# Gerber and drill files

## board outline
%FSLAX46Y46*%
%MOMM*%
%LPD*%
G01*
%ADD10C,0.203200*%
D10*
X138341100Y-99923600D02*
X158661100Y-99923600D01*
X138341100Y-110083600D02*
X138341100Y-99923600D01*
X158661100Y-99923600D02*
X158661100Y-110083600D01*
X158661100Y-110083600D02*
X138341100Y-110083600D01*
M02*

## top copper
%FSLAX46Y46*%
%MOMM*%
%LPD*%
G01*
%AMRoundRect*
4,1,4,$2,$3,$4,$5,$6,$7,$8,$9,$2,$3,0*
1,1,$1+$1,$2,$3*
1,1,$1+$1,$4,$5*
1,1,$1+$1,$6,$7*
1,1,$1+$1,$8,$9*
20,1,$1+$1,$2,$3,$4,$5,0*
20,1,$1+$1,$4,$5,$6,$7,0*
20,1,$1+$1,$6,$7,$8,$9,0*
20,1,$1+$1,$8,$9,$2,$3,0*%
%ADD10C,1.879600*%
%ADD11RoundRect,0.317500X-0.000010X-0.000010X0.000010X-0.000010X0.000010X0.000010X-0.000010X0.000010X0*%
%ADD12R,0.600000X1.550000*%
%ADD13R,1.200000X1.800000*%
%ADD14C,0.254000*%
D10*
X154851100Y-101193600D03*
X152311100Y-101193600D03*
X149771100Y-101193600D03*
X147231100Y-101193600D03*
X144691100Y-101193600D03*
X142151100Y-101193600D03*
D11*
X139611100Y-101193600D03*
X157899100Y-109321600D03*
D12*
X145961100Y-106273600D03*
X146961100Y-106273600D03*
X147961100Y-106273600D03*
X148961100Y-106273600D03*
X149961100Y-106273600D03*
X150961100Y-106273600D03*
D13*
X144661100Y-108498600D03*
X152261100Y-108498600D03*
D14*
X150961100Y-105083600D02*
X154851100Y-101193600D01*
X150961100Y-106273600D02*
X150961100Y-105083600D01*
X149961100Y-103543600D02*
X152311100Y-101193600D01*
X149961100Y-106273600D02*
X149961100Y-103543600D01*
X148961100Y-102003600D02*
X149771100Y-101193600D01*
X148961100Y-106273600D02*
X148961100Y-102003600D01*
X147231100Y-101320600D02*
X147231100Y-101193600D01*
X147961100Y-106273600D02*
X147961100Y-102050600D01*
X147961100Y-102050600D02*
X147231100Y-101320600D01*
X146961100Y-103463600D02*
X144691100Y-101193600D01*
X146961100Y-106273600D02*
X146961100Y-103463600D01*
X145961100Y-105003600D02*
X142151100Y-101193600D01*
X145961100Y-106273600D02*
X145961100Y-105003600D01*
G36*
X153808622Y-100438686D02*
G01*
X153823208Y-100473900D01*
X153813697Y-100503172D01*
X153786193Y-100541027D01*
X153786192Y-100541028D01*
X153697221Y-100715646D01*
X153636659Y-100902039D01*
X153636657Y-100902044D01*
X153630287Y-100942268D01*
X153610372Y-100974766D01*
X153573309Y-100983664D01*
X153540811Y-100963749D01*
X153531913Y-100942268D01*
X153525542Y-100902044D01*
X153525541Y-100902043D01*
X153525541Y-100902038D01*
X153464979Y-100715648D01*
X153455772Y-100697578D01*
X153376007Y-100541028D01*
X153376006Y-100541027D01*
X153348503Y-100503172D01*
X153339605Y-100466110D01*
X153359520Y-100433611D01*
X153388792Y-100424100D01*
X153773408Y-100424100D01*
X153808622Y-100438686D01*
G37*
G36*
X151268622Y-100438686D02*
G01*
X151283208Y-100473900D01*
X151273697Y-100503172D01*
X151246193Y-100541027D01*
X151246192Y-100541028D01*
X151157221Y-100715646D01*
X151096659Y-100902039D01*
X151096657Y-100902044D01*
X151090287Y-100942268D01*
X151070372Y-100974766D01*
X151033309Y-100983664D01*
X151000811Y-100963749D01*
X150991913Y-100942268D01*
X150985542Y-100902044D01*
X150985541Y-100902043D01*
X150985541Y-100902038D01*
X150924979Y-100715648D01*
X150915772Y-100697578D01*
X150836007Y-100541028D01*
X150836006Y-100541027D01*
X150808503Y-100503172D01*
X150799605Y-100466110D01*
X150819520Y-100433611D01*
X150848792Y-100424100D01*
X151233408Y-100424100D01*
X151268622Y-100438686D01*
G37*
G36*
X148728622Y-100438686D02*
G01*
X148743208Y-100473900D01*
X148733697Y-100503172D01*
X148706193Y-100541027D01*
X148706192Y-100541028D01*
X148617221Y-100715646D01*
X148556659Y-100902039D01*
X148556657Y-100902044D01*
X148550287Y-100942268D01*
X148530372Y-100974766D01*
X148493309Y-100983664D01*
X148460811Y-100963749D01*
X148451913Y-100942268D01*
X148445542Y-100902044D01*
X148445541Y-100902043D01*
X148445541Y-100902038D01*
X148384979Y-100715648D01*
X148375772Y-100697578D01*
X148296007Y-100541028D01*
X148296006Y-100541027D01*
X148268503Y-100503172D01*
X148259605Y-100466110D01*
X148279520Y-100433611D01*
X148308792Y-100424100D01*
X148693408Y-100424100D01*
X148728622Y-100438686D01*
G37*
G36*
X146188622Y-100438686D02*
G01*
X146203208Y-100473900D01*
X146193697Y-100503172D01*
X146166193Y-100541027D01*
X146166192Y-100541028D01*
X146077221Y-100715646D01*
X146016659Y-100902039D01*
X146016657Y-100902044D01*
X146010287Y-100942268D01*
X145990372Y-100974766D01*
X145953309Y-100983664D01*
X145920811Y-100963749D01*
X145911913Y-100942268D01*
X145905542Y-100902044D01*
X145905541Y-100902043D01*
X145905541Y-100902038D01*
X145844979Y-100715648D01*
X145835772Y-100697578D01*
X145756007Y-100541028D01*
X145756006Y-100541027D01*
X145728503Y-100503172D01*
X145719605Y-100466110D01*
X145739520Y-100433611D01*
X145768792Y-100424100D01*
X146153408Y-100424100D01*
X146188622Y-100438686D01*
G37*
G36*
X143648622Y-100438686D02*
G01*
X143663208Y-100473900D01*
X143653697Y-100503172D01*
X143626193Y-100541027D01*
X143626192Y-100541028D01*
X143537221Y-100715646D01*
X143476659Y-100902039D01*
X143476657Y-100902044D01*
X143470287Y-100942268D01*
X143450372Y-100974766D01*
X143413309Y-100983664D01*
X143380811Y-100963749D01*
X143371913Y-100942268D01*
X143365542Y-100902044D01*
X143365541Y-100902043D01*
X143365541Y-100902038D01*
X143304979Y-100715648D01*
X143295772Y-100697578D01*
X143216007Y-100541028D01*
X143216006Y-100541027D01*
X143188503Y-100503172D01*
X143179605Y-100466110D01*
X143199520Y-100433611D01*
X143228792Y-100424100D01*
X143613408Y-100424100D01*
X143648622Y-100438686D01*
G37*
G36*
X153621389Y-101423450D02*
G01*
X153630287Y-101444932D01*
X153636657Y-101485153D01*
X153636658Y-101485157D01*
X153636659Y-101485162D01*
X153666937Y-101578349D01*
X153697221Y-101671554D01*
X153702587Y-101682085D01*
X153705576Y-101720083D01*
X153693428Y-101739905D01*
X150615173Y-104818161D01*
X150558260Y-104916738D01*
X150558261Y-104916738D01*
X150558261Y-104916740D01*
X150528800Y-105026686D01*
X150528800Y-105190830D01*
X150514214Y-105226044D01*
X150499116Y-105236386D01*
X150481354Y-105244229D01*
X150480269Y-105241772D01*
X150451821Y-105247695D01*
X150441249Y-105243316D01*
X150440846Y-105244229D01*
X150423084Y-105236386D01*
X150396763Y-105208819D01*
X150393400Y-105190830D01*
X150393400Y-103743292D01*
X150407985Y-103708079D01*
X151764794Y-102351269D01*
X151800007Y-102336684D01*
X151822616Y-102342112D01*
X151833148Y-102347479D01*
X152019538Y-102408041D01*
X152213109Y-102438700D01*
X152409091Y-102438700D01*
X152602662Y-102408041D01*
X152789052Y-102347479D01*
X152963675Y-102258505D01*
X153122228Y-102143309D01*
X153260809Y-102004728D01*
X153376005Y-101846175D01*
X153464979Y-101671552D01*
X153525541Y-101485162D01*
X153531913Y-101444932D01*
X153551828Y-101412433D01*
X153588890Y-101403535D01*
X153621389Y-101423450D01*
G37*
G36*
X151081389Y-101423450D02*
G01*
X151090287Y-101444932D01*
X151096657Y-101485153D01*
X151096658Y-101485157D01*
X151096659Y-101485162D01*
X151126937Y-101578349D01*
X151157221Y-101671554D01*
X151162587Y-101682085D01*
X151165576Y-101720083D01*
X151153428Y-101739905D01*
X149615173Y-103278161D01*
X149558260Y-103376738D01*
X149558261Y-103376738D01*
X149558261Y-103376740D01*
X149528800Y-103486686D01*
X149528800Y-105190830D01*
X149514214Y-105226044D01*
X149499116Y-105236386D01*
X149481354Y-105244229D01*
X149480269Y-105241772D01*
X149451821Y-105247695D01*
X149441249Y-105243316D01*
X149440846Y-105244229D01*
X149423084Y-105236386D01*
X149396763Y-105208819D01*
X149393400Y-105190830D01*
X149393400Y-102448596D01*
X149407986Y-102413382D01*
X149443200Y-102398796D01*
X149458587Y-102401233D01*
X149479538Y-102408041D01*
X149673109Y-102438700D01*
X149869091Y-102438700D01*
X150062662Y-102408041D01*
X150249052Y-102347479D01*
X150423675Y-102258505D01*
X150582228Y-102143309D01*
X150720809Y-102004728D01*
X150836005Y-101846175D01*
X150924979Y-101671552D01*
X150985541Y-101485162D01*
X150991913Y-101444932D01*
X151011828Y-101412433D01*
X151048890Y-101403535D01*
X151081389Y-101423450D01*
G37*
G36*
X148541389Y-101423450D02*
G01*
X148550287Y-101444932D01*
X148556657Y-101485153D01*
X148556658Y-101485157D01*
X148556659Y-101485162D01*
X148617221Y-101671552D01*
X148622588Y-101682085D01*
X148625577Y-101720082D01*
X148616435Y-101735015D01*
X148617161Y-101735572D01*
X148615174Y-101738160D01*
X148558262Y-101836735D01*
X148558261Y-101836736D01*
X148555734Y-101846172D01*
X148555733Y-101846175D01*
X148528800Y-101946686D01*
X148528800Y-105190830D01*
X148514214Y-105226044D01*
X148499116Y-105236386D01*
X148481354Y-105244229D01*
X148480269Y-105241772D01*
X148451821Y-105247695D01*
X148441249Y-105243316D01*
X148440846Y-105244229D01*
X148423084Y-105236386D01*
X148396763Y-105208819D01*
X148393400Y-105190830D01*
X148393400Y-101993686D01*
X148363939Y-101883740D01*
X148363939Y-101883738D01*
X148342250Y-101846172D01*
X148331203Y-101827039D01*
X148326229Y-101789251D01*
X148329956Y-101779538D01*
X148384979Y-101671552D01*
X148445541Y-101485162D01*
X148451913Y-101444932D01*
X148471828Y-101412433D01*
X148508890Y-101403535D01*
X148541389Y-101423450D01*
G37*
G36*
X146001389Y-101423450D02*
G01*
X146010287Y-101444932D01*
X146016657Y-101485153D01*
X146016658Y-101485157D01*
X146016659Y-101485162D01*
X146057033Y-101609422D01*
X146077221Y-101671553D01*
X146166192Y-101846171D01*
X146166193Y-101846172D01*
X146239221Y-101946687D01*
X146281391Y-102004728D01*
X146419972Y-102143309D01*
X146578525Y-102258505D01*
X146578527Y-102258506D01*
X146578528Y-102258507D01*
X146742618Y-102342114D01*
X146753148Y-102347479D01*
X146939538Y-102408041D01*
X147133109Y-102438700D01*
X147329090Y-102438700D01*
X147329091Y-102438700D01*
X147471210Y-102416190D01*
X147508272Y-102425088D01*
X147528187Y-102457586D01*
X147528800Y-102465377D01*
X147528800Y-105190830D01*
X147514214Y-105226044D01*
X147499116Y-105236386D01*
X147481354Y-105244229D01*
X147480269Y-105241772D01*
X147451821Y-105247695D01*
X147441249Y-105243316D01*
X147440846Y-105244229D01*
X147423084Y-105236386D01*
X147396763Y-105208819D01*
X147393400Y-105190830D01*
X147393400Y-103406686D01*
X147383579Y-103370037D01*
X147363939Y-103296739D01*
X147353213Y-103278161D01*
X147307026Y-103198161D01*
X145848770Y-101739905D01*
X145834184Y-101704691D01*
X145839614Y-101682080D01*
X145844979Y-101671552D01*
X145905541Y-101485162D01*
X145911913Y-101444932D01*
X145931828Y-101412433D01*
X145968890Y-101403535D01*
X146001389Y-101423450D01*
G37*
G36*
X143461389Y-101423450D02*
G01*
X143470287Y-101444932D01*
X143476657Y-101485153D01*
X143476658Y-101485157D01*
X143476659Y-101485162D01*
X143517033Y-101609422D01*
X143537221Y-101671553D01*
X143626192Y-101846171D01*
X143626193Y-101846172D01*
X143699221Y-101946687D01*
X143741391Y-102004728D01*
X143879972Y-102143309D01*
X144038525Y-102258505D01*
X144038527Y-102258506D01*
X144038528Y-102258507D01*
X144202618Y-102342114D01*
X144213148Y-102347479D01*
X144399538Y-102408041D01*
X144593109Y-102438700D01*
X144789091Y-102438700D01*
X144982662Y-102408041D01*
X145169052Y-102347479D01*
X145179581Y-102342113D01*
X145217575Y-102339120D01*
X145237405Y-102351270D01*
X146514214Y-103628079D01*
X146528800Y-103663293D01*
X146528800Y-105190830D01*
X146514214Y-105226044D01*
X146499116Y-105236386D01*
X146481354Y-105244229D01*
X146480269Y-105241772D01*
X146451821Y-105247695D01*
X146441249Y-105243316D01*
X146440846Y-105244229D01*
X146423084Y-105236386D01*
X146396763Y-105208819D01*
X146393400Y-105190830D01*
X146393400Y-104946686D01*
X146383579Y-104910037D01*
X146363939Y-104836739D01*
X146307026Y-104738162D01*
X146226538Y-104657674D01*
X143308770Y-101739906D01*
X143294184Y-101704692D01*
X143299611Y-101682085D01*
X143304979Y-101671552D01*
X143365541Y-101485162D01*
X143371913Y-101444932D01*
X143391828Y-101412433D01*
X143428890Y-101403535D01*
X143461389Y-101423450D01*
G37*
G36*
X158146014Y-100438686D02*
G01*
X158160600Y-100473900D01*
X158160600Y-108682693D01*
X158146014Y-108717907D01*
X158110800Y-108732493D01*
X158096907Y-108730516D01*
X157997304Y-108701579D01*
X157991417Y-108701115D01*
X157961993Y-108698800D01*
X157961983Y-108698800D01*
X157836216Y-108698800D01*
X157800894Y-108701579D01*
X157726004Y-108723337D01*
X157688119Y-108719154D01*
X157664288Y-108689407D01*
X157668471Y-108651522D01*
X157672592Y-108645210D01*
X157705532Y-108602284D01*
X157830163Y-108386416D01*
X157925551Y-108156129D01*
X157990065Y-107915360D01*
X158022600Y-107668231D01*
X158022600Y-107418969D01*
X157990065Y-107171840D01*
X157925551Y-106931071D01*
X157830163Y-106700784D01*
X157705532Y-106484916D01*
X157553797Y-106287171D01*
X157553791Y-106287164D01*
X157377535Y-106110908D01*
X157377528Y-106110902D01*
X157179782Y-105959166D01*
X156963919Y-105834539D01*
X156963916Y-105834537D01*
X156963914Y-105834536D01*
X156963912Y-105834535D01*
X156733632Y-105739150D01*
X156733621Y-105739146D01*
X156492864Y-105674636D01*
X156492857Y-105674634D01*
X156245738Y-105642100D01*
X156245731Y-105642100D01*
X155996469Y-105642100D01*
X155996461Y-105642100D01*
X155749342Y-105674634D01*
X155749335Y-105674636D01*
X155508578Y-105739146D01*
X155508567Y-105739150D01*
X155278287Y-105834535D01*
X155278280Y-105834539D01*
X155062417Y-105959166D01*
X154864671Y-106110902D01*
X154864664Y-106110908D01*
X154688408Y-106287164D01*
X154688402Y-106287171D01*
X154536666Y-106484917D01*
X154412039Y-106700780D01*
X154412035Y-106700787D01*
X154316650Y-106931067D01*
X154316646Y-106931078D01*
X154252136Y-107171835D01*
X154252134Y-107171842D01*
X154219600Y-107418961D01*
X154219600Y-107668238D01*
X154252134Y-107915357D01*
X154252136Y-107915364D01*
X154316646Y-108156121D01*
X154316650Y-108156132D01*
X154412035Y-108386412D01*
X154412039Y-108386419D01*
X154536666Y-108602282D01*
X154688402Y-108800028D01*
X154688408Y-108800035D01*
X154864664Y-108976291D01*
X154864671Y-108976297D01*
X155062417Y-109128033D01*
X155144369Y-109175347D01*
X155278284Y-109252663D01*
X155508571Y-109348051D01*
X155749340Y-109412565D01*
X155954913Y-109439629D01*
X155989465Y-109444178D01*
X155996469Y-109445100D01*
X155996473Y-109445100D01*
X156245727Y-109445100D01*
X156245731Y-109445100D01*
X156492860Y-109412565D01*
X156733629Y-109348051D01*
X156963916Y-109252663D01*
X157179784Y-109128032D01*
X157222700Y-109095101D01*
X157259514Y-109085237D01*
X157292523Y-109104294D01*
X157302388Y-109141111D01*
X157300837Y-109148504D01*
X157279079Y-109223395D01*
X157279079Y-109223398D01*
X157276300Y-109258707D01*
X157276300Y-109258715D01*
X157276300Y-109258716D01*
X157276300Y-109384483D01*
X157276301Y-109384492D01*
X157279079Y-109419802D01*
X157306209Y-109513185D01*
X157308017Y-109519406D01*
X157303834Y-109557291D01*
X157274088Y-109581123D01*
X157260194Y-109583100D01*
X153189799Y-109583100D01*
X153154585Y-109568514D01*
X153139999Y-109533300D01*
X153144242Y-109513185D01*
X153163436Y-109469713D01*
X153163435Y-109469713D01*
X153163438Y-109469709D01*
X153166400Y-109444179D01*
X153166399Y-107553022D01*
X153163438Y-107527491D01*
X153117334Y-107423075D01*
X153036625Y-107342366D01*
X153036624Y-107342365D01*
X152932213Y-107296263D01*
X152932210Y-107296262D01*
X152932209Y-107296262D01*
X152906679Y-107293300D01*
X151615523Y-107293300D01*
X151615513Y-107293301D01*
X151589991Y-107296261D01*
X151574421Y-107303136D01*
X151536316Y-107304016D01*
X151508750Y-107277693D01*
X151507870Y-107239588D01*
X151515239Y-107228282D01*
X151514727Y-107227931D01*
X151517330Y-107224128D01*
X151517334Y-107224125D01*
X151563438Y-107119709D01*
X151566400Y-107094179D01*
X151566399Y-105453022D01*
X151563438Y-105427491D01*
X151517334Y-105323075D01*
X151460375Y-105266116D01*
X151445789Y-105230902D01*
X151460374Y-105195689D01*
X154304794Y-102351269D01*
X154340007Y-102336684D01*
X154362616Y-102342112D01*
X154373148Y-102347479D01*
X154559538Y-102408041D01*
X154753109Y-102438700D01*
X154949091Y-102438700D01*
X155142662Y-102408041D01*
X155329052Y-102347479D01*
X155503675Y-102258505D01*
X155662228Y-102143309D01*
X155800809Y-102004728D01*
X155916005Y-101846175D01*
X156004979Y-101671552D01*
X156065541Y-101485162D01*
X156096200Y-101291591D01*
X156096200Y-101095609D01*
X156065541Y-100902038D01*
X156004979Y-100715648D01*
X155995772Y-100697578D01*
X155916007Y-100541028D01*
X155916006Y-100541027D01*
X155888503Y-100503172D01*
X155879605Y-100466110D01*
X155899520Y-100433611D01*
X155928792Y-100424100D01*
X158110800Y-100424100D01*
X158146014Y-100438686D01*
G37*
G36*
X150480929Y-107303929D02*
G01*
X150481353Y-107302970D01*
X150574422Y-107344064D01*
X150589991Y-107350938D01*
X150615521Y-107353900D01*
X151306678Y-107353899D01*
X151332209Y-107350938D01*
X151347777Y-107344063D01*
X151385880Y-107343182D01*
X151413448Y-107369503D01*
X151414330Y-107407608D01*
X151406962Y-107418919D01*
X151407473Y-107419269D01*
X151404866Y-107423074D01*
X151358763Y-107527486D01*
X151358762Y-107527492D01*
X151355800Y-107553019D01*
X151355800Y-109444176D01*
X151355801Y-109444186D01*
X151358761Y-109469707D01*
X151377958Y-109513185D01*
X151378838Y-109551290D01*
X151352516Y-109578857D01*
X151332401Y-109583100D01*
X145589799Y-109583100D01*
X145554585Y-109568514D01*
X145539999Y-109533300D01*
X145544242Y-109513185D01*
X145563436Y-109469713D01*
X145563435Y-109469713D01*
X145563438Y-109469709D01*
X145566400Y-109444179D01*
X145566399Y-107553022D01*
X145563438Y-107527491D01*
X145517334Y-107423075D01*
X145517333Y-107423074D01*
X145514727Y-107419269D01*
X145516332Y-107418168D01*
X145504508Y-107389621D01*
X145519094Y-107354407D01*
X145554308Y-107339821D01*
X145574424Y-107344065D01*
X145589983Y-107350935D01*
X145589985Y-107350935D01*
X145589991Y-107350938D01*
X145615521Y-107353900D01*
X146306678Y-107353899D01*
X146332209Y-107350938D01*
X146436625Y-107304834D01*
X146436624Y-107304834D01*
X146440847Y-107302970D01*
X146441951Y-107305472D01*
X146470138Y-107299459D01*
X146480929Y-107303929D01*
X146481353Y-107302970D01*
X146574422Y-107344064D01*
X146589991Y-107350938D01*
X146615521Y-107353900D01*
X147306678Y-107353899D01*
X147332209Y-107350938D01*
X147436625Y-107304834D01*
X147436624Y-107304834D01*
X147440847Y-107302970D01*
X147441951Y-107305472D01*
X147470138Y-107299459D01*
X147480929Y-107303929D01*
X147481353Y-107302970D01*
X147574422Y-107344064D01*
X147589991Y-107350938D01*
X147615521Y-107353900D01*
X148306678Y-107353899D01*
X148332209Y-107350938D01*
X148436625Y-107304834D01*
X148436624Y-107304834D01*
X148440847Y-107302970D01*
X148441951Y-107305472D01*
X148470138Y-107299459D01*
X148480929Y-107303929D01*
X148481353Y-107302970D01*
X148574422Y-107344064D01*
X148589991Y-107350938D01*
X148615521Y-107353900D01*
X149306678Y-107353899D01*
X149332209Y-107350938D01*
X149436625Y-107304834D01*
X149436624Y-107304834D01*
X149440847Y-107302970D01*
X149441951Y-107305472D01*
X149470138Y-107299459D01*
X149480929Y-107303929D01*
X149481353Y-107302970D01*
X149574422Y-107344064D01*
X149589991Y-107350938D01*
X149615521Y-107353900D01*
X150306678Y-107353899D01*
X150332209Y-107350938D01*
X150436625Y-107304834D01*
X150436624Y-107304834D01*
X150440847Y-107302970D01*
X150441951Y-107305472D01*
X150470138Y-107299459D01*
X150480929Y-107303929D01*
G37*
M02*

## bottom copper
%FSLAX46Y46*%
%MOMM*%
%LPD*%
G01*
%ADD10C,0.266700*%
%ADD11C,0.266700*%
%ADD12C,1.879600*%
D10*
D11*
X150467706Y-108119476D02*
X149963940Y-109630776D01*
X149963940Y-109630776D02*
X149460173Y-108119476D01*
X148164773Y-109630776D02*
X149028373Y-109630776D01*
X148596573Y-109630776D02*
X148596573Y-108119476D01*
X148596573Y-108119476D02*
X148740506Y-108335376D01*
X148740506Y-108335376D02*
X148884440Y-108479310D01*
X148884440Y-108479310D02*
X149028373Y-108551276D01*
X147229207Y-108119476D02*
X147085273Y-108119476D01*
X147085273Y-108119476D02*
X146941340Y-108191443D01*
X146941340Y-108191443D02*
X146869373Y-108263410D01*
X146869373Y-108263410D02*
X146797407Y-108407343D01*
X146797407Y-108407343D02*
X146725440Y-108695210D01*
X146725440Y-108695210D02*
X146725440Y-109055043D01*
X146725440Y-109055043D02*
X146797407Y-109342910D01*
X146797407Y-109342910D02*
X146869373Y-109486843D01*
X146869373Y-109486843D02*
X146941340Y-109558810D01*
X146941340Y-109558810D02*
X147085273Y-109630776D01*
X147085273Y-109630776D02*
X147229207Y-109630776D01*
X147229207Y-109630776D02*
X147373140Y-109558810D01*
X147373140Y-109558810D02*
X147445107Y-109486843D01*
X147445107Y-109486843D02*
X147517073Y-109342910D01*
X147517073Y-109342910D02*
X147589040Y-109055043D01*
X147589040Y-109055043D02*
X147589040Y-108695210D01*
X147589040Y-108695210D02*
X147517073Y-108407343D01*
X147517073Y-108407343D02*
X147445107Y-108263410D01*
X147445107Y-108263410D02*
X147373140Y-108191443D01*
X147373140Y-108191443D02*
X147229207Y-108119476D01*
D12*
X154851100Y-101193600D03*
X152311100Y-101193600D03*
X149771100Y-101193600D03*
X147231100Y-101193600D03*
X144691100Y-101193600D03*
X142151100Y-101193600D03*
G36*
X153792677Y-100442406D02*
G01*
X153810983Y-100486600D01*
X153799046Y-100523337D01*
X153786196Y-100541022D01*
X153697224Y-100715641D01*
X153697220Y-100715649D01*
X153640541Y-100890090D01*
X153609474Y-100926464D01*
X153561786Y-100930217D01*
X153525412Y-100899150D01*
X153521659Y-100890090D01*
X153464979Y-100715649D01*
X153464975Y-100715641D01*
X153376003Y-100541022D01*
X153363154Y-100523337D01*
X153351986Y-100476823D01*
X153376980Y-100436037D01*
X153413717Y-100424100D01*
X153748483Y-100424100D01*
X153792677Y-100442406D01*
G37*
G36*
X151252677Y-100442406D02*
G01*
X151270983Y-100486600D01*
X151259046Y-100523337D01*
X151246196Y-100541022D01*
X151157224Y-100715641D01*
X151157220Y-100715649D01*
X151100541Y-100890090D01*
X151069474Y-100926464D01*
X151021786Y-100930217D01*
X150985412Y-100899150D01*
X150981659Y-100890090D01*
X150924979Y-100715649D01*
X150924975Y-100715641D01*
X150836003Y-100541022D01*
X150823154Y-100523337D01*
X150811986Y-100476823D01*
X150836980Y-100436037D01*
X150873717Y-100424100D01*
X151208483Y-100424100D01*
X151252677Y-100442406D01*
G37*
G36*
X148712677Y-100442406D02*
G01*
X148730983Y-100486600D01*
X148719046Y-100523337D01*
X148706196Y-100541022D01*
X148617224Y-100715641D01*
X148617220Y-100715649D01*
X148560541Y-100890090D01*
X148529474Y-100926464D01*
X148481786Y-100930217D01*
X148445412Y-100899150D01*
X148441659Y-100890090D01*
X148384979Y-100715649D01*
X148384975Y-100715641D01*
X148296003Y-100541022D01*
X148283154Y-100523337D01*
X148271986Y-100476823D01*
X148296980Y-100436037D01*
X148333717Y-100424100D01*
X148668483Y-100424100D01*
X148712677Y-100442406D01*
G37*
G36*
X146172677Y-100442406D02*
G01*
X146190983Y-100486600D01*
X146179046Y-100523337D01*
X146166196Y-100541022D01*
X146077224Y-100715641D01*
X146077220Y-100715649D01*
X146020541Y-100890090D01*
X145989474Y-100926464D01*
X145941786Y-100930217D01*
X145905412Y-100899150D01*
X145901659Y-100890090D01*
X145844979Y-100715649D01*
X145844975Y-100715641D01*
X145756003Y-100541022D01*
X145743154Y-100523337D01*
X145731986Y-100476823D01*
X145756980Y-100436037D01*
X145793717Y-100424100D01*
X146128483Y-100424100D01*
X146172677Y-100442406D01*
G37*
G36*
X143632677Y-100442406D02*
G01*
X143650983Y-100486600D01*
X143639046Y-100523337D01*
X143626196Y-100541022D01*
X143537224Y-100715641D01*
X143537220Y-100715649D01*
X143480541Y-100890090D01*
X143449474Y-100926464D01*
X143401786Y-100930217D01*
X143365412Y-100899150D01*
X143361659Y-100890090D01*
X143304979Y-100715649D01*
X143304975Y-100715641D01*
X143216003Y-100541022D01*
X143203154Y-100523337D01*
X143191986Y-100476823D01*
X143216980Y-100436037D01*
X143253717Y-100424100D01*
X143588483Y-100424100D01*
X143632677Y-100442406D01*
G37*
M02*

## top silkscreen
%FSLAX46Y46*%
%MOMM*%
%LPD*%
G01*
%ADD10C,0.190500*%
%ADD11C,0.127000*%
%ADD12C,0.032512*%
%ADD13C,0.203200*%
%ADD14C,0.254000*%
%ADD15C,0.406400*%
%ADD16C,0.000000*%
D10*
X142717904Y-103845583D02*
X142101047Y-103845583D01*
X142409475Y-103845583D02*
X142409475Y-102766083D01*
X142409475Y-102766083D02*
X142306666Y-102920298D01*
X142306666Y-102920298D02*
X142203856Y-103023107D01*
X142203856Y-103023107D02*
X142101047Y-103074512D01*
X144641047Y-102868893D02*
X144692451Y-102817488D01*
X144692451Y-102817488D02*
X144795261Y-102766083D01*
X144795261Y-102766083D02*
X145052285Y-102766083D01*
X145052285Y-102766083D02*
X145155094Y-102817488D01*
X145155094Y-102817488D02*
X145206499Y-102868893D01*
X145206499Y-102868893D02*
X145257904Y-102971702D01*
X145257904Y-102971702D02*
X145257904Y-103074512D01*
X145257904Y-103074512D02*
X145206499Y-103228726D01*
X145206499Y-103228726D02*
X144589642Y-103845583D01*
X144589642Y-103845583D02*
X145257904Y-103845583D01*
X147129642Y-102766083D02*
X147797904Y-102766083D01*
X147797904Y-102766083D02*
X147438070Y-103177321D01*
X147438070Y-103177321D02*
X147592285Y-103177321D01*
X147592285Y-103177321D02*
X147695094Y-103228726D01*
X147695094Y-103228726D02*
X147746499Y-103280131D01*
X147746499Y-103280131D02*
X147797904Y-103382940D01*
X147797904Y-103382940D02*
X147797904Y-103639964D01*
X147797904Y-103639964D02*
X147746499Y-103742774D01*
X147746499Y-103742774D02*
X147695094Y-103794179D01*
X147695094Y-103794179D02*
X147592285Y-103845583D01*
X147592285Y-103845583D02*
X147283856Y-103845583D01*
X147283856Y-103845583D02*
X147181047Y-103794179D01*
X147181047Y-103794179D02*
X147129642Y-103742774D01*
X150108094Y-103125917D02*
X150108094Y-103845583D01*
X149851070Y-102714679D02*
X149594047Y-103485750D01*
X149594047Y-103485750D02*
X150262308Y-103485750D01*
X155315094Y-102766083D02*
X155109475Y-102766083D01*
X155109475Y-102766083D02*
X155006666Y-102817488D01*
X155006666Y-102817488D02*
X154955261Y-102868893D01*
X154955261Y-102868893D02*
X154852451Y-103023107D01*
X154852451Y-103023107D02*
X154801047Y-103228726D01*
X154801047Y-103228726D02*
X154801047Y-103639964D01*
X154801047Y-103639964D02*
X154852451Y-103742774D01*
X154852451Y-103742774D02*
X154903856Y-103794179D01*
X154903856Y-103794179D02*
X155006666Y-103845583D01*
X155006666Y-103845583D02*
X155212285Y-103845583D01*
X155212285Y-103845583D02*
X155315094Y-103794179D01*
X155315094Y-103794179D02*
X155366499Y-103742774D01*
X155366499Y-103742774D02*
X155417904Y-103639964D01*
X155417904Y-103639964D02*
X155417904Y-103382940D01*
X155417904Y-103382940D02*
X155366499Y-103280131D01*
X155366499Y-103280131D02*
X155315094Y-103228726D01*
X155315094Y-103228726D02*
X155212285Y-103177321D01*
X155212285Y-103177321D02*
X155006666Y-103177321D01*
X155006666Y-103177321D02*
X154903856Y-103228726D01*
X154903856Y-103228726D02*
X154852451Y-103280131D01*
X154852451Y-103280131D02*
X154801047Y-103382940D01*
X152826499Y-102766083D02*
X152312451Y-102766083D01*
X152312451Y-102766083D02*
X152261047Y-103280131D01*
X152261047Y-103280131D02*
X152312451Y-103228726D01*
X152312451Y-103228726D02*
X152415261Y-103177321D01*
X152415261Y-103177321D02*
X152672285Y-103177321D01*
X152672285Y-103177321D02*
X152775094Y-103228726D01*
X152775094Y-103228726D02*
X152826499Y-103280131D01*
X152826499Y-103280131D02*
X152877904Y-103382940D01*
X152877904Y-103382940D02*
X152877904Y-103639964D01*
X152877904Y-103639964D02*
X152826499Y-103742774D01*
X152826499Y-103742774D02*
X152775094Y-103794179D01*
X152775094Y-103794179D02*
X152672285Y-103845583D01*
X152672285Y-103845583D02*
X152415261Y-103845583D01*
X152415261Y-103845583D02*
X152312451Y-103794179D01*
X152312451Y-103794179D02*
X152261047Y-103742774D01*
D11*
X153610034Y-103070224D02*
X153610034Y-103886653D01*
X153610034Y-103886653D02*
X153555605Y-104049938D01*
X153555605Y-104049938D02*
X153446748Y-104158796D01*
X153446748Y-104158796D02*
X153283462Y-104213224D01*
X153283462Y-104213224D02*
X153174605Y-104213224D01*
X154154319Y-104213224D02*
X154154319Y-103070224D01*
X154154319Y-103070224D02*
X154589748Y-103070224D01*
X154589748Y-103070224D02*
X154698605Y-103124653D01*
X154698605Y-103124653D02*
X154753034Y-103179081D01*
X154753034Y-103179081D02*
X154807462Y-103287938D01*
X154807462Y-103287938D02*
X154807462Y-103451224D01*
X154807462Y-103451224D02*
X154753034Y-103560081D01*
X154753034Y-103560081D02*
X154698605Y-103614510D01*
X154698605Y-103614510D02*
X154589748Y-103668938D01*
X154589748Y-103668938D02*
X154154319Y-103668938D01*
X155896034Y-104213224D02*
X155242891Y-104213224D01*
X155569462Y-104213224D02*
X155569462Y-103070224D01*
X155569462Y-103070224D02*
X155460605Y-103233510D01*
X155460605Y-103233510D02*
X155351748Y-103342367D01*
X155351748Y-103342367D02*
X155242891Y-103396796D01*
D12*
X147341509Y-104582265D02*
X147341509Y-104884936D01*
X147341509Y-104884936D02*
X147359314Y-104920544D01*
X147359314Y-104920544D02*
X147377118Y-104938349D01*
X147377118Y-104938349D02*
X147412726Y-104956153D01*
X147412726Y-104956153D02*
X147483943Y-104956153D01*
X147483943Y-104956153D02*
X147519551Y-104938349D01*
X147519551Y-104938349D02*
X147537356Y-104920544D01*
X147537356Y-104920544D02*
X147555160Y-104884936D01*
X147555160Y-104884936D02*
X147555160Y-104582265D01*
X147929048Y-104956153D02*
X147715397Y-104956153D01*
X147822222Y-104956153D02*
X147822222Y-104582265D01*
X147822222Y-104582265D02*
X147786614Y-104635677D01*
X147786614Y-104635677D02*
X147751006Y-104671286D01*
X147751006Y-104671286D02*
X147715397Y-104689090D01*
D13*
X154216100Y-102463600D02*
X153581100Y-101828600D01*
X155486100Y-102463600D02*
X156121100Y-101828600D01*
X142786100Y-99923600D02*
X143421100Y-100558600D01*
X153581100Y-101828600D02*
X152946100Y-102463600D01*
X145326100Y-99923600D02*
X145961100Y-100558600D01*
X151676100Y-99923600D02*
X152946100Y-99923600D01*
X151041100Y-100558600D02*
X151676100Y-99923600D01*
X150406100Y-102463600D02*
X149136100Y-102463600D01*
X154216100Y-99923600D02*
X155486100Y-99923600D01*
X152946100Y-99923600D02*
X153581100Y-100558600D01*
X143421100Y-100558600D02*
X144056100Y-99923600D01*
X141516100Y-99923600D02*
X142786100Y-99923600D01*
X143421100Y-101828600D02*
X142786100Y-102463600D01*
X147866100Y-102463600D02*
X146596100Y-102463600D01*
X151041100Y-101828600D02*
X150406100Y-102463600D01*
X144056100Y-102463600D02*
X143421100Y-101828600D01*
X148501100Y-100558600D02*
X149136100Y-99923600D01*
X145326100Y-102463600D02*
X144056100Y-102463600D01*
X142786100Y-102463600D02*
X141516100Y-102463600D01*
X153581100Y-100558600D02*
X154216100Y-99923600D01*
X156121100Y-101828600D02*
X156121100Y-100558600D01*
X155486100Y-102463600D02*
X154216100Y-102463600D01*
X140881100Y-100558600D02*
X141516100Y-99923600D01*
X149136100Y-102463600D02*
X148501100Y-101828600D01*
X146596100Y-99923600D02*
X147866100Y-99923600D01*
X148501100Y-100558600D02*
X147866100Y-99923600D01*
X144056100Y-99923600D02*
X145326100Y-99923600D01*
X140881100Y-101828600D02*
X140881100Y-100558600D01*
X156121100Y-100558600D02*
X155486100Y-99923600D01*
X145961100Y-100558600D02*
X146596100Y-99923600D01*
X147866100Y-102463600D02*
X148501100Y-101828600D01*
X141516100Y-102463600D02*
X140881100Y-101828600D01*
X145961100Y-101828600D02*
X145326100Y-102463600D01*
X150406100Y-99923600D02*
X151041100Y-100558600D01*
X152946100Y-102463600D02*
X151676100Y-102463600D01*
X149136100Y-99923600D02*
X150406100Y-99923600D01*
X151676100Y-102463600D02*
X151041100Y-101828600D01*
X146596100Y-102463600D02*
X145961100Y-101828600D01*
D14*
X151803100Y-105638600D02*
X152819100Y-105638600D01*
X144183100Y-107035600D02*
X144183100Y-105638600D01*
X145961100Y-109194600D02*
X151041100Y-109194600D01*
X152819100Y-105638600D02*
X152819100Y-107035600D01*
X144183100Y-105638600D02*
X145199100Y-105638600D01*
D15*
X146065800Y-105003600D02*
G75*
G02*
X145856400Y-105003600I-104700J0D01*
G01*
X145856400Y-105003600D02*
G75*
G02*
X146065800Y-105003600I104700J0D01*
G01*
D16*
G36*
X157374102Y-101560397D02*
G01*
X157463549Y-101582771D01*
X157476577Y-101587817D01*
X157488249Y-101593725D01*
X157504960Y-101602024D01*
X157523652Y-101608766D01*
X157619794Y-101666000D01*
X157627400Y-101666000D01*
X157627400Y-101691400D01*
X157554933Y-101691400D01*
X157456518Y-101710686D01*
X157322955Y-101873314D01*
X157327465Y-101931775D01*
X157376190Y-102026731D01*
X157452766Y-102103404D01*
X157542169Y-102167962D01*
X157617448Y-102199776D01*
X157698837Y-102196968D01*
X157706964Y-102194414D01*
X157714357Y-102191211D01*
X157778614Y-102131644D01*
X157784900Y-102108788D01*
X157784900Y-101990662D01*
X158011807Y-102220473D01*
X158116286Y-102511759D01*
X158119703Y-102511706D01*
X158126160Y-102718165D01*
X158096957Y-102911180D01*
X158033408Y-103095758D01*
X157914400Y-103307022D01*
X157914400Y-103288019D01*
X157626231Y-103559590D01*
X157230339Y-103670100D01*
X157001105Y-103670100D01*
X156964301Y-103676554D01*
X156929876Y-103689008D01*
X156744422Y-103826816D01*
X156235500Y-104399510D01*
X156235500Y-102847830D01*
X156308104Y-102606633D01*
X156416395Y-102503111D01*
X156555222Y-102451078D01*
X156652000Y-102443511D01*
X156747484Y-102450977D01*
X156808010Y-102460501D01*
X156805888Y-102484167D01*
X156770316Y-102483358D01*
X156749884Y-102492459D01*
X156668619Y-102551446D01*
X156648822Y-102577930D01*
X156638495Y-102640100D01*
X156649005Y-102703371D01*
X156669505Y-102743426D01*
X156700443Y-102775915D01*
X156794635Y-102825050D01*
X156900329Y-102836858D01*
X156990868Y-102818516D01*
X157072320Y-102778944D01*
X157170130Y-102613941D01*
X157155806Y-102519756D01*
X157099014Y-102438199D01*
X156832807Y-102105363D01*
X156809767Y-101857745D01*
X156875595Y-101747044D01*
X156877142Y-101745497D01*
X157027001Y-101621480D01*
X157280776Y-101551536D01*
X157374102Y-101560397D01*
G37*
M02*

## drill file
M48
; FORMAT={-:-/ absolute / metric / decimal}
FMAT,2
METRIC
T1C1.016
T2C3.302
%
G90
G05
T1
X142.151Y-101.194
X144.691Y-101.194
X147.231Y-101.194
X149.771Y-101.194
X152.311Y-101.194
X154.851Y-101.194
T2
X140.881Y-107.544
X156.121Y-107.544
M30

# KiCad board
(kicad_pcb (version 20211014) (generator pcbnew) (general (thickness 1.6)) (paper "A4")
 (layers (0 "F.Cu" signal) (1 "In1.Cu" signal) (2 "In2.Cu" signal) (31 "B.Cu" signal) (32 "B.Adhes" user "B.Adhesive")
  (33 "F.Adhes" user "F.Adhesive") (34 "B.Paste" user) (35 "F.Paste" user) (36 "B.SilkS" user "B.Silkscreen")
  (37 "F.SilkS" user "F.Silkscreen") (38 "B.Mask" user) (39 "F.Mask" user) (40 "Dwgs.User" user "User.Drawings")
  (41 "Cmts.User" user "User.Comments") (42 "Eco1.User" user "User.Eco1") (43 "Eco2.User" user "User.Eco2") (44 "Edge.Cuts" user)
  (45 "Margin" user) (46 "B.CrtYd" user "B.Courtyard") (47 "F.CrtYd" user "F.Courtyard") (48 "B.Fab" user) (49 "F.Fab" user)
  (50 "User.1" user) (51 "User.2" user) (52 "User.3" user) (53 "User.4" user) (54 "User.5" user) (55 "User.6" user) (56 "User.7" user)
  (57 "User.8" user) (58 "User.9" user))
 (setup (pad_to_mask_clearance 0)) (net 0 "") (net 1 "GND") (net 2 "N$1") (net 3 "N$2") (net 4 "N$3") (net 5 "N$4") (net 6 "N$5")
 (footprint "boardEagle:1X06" (layer "F.Cu") (at 154.8511 101.1936 180)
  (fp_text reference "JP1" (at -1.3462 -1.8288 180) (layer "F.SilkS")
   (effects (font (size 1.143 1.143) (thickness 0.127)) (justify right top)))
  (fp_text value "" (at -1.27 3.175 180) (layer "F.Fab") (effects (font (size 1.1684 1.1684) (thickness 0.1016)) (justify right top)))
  (fp_line (start 0.635 -1.27) (end 1.27 -0.635) (layer "F.SilkS") (width 0.2032))
  (fp_line (start -0.635 -1.27) (end -1.27 -0.635) (layer "F.SilkS") (width 0.2032))
  (fp_line (start 12.065 1.27) (end 11.43 0.635) (layer "F.SilkS") (width 0.2032))
  (fp_line (start 1.27 -0.635) (end 1.905 -1.27) (layer "F.SilkS") (width 0.2032))
  (fp_line (start 9.525 1.27) (end 8.89 0.635) (layer "F.SilkS") (width 0.2032))
  (fp_line (start 3.175 1.27) (end 1.905 1.27) (layer "F.SilkS") (width 0.2032))
  (fp_line (start 3.81 0.635) (end 3.175 1.27) (layer "F.SilkS") (width 0.2032))
  (fp_line (start 4.445 -1.27) (end 5.715 -1.27) (layer "F.SilkS") (width 0.2032))
  (fp_line (start 0.635 1.27) (end -0.635 1.27) (layer "F.SilkS") (width 0.2032))
  (fp_line (start 1.905 1.27) (end 1.27 0.635) (layer "F.SilkS") (width 0.2032))
  (fp_line (start 11.43 0.635) (end 10.795 1.27) (layer "F.SilkS") (width 0.2032))
  (fp_line (start 13.335 1.27) (end 12.065 1.27) (layer "F.SilkS") (width 0.2032))
  (fp_line (start 11.43 -0.635) (end 12.065 -1.27) (layer "F.SilkS") (width 0.2032))
  (fp_line (start 6.985 -1.27) (end 8.255 -1.27) (layer "F.SilkS") (width 0.2032))
  (fp_line (start 3.81 -0.635) (end 4.445 -1.27) (layer "F.SilkS") (width 0.2032))
  (fp_line (start 10.795 -1.27) (end 11.43 -0.635) (layer "F.SilkS") (width 0.2032))
  (fp_line (start 6.35 0.635) (end 5.715 1.27) (layer "F.SilkS") (width 0.2032))
  (fp_line (start 9.525 -1.27) (end 10.795 -1.27) (layer "F.SilkS") (width 0.2032))
  (fp_line (start 12.065 -1.27) (end 13.335 -1.27) (layer "F.SilkS") (width 0.2032))
  (fp_line (start 1.27 0.635) (end 0.635 1.27) (layer "F.SilkS") (width 0.2032))
  (fp_line (start -1.27 -0.635) (end -1.27 0.635) (layer "F.SilkS") (width 0.2032))
  (fp_line (start -0.635 -1.27) (end 0.635 -1.27) (layer "F.SilkS") (width 0.2032))
  (fp_line (start 13.97 0.635) (end 13.335 1.27) (layer "F.SilkS") (width 0.2032))
  (fp_line (start 5.715 -1.27) (end 6.35 -0.635) (layer "F.SilkS") (width 0.2032))
  (fp_line (start 8.255 1.27) (end 6.985 1.27) (layer "F.SilkS") (width 0.2032))
  (fp_line (start 6.35 0.635) (end 6.985 1.27) (layer "F.SilkS") (width 0.2032))
  (fp_line (start 10.795 1.27) (end 9.525 1.27) (layer "F.SilkS") (width 0.2032))
  (fp_line (start 13.97 -0.635) (end 13.97 0.635) (layer "F.SilkS") (width 0.2032))
  (fp_line (start -1.27 0.635) (end -0.635 1.27) (layer "F.SilkS") (width 0.2032))
  (fp_line (start 8.89 0.635) (end 8.255 1.27) (layer "F.SilkS") (width 0.2032))
  (fp_line (start 6.985 -1.27) (end 6.35 -0.635) (layer "F.SilkS") (width 0.2032))
  (fp_line (start 13.335 -1.27) (end 13.97 -0.635) (layer "F.SilkS") (width 0.2032))
  (fp_line (start 8.89 -0.635) (end 9.525 -1.27) (layer "F.SilkS") (width 0.2032))
  (fp_line (start 4.445 1.27) (end 3.81 0.635) (layer "F.SilkS") (width 0.2032))
  (fp_line (start 1.905 -1.27) (end 3.175 -1.27) (layer "F.SilkS") (width 0.2032))
  (fp_line (start 5.715 1.27) (end 4.445 1.27) (layer "F.SilkS") (width 0.2032))
  (fp_line (start 3.175 -1.27) (end 3.81 -0.635) (layer "F.SilkS") (width 0.2032))
  (fp_line (start 8.255 -1.27) (end 8.89 -0.635) (layer "F.SilkS") (width 0.2032))
  (pad "1" thru_hole circle (at 0 0 270) (size 1.8796 1.8796) (drill 1.016) (layers *.Cu *.Mask) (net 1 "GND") (solder_mask_margin 0.1016))
  (pad "2" thru_hole circle (at 2.54 0 270) (size 1.8796 1.8796) (drill 1.016) (layers *.Cu *.Mask) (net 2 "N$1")
   (solder_mask_margin 0.1016))
  (pad "3" thru_hole circle (at 5.08 0 270) (size 1.8796 1.8796) (drill 1.016) (layers *.Cu *.Mask) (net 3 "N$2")
   (solder_mask_margin 0.1016))
  (pad "4" thru_hole circle (at 7.62 0 270) (size 1.8796 1.8796) (drill 1.016) (layers *.Cu *.Mask) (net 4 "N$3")
   (solder_mask_margin 0.1016))
  (pad "5" thru_hole circle (at 10.16 0 270) (size 1.8796 1.8796) (drill 1.016) (layers *.Cu *.Mask) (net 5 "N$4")
   (solder_mask_margin 0.1016))
  (pad "6" thru_hole circle (at 12.7 0 270) (size 1.8796 1.8796) (drill 1.016) (layers *.Cu *.Mask) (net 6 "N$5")
   (solder_mask_margin 0.1016)))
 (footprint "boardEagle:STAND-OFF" (layer "F.Cu") (at 140.8811 107.5436)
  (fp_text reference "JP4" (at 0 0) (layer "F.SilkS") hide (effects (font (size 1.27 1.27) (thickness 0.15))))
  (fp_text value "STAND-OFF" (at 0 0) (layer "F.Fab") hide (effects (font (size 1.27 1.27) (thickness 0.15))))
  (pad "" np_thru_hole circle (at 0 0) (size 3.302 3.302) (drill 3.302) (layers *.Cu *.Mask)))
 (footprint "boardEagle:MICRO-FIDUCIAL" (layer "F.Cu") (at 139.6111 101.1936)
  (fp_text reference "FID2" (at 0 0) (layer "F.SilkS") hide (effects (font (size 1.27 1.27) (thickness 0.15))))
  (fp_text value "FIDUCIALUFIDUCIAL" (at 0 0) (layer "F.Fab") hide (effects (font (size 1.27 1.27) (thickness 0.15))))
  (pad "1" smd roundrect (at 0 0) (size 0.635 0.635) (layers "F.Cu" "F.Mask") (roundrect_rratio 0.5) (solder_mask_margin 0.1016)))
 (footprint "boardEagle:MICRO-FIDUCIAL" (layer "F.Cu") (at 157.8991 109.3216)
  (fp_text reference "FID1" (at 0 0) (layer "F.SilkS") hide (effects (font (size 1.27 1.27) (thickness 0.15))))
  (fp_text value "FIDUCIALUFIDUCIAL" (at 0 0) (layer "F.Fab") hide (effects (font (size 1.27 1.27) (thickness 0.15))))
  (pad "1" smd roundrect (at 0 0) (size 0.635 0.635) (layers "F.Cu" "F.Mask") (roundrect_rratio 0.5) (solder_mask_margin 0.1016)))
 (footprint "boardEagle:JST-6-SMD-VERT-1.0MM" (layer "F.Cu") (at 148.5011 107.5436)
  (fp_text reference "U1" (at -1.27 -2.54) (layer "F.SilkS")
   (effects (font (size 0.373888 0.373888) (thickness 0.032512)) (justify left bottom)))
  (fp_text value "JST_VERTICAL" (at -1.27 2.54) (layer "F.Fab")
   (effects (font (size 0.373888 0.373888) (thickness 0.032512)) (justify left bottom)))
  (fp_line (start 3.302 -1.905) (end 4.318 -1.905) (layer "F.SilkS") (width 0.254))
  (fp_line (start -4.318 -0.508) (end -4.318 -1.905) (layer "F.SilkS") (width 0.254))
  (fp_line (start -2.54 1.651) (end 2.54 1.651) (layer "F.SilkS") (width 0.254))
  (fp_line (start 4.318 -1.905) (end 4.318 -0.508) (layer "F.SilkS") (width 0.254))
  (fp_line (start -4.318 -1.905) (end -3.302 -1.905) (layer "F.SilkS") (width 0.254))
  (fp_circle (center -2.54 -2.54) (end -2.4353 -2.54) (layer "F.SilkS") (width 0.4064) (fill none))
  (pad "1" smd rect (at -2.54 -1.27) (size 0.6 1.55) (layers "F.Cu" "F.Paste" "F.Mask") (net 6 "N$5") (solder_mask_margin 0.1016))
  (pad "2" smd rect (at -1.54 -1.27) (size 0.6 1.55) (layers "F.Cu" "F.Paste" "F.Mask") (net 5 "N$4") (solder_mask_margin 0.1016))
  (pad "3" smd rect (at -0.54 -1.27) (size 0.6 1.55) (layers "F.Cu" "F.Paste" "F.Mask") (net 4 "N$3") (solder_mask_margin 0.1016))
  (pad "4" smd rect (at 0.46 -1.27) (size 0.6 1.55) (layers "F.Cu" "F.Paste" "F.Mask") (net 3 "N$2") (solder_mask_margin 0.1016))
  (pad "5" smd rect (at 1.46 -1.27) (size 0.6 1.55) (layers "F.Cu" "F.Paste" "F.Mask") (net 2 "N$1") (solder_mask_margin 0.1016))
  (pad "6" smd rect (at 2.46 -1.27) (size 0.6 1.55) (layers "F.Cu" "F.Paste" "F.Mask") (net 1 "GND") (solder_mask_margin 0.1016))
  (pad "P$1" smd rect (at -3.84 0.955) (size 1.2 1.8) (layers "F.Cu" "F.Paste" "F.Mask") (solder_mask_margin 0.1016))
  (pad "P$2" smd rect (at 3.76 0.955) (size 1.2 1.8) (layers "F.Cu" "F.Paste" "F.Mask") (solder_mask_margin 0.1016)))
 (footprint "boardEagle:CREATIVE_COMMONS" (layer "F.Cu") (at 157.3911 118.9736)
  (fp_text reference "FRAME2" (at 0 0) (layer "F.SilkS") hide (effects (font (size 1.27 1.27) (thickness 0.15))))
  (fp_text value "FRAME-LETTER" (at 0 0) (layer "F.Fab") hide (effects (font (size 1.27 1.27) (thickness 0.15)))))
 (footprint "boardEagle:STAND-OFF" (layer "F.Cu") (at 156.1211 107.5436)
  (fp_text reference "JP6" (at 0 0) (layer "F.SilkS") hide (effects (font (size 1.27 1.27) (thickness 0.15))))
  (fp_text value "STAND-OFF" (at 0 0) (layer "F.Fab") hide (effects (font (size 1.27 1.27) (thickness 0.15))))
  (pad "" np_thru_hole circle (at 0 0) (size 3.302 3.302) (drill 3.302) (layers *.Cu *.Mask)))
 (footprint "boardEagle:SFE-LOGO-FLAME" (layer "F.Cu") (at 156.2481 104.3686)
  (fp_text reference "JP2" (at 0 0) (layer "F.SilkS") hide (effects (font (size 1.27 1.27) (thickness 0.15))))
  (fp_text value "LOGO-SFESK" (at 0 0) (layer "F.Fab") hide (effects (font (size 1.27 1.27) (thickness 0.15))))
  (fp_poly
   (pts (xy 1.126002 -2.808203) (xy 1.215449 -2.785829) (xy 1.228477 -2.780783) (xy 1.240149 -2.774875) (xy 1.25686 -2.766576)
    (xy 1.275552 -2.759834) (xy 1.371694 -2.7026) (xy 1.3793 -2.7026) (xy 1.3793 -2.6772) (xy 1.306833 -2.6772) (xy 1.208418 -2.657914)
    (xy 1.074855 -2.495286) (xy 1.079365 -2.436825) (xy 1.12809 -2.341869) (xy 1.204666 -2.265196) (xy 1.294069 -2.200638)
    (xy 1.369348 -2.168824) (xy 1.450737 -2.171632) (xy 1.458864 -2.174186) (xy 1.466257 -2.177389) (xy 1.530514 -2.236956)
    (xy 1.5368 -2.259812) (xy 1.5368 -2.377938) (xy 1.763707 -2.148127) (xy 1.868186 -1.856841) (xy 1.871603 -1.856894)
    (xy 1.87806 -1.650435) (xy 1.848857 -1.45742) (xy 1.785308 -1.272842) (xy 1.6663 -1.061578) (xy 1.6663 -1.080581) (xy 1.378131 -0.80901)
    (xy 0.982239 -0.6985) (xy 0.753005 -0.6985) (xy 0.716201 -0.692046) (xy 0.681776 -0.679592) (xy 0.496322 -0.541784) (xy -0.0126 0.03091)
    (xy -0.0126 -1.52077) (xy 0.060004 -1.761967) (xy 0.168295 -1.865489) (xy 0.307122 -1.917522) (xy 0.4039 -1.925089)
    (xy 0.499384 -1.917623) (xy 0.55991 -1.908099) (xy 0.557788 -1.884433) (xy 0.522216 -1.885242) (xy 0.501784 -1.876141)
    (xy 0.420519 -1.817154) (xy 0.400722 -1.79067) (xy 0.390395 -1.7285) (xy 0.400905 -1.665229) (xy 0.421405 -1.625174)
    (xy 0.452343 -1.592685) (xy 0.546535 -1.54355) (xy 0.652229 -1.531742) (xy 0.742768 -1.550084) (xy 0.82422 -1.589656)
    (xy 0.92203 -1.754659) (xy 0.907706 -1.848844) (xy 0.850914 -1.930401) (xy 0.584707 -2.263237) (xy 0.561667 -2.510855)
    (xy 0.627495 -2.621556) (xy 0.629042 -2.623103) (xy 0.778901 -2.74712) (xy 1.032676 -2.817064))
   (layer "F.SilkS") (width 0) (fill solid)))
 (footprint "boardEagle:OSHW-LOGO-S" (layer "B.Cu") (at 156.7561 104.1146 180)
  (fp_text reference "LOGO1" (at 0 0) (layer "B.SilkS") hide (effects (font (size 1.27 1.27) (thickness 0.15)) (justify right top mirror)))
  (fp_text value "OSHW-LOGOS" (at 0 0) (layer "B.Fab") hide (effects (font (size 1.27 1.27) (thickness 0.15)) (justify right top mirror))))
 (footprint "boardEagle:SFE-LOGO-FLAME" (layer "B.Cu") (at 140.8811 105.0036 180)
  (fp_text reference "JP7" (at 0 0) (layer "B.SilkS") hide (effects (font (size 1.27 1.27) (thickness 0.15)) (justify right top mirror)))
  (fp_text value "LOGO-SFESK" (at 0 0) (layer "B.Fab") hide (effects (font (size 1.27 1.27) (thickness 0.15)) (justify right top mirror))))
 (gr_line (start 138.3411 99.9236) (end 158.6611 99.9236) (layer "Edge.Cuts") (width 0.2032))
 (gr_line (start 138.3411 110.0836) (end 138.3411 99.9236) (layer "Edge.Cuts") (width 0.2032))
 (gr_line (start 158.6611 99.9236) (end 158.6611 110.0836) (layer "Edge.Cuts") (width 0.2032))
 (gr_line (start 158.6611 110.0836) (end 138.3411 110.0836) (layer "Edge.Cuts") (width 0.2032))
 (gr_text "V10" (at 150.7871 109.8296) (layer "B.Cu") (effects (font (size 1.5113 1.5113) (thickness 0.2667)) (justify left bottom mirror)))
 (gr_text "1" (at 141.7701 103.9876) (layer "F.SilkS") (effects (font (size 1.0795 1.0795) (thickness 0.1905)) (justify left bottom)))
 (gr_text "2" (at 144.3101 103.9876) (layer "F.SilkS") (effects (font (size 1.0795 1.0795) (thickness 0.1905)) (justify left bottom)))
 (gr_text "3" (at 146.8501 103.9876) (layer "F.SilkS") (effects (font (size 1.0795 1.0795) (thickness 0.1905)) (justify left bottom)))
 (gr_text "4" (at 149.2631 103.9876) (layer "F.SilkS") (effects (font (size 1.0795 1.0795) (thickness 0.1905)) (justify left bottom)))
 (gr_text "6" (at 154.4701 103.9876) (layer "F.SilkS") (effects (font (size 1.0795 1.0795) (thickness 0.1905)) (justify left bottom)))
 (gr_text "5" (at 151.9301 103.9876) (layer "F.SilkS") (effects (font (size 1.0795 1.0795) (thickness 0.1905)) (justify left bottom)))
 (segment (start 150.9611 105.0836) (end 154.8511 101.1936) (width 0.254) (layer "F.Cu") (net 1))
 (segment (start 150.9611 106.2736) (end 150.9611 105.0836) (width 0.254) (layer "F.Cu") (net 1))
 (segment (start 149.9611 103.5436) (end 152.3111 101.1936) (width 0.254) (layer "F.Cu") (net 2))
 (segment (start 149.9611 106.2736) (end 149.9611 103.5436) (width 0.254) (layer "F.Cu") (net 2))
 (segment (start 148.9611 102.0036) (end 149.7711 101.1936) (width 0.254) (layer "F.Cu") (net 3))
 (segment (start 148.9611 106.2736) (end 148.9611 102.0036) (width 0.254) (layer "F.Cu") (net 3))
 (segment (start 147.2311 101.3206) (end 147.2311 101.1936) (width 0.254) (layer "F.Cu") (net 4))
 (segment (start 147.9611 106.2736) (end 147.9611 102.0506) (width 0.254) (layer "F.Cu") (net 4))
 (segment (start 147.9611 102.0506) (end 147.2311 101.3206) (width 0.254) (layer "F.Cu") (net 4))
 (segment (start 146.9611 103.4636) (end 144.6911 101.1936) (width 0.254) (layer "F.Cu") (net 5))
 (segment (start 146.9611 106.2736) (end 146.9611 103.4636) (width 0.254) (layer "F.Cu") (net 5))
 (segment (start 145.9611 105.0036) (end 142.1511 101.1936) (width 0.254) (layer "F.Cu") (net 6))
 (segment (start 145.9611 106.2736) (end 145.9611 105.0036) (width 0.254) (layer "F.Cu") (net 6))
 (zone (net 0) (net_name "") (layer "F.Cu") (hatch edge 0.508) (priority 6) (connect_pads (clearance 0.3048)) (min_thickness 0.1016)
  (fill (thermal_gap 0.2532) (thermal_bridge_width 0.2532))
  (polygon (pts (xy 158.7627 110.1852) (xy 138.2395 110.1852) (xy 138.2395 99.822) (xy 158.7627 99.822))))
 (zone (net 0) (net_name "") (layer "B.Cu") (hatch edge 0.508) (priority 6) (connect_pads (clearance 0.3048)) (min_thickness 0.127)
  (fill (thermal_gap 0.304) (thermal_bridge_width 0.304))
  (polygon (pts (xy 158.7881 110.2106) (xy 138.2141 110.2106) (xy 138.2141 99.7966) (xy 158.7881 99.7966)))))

